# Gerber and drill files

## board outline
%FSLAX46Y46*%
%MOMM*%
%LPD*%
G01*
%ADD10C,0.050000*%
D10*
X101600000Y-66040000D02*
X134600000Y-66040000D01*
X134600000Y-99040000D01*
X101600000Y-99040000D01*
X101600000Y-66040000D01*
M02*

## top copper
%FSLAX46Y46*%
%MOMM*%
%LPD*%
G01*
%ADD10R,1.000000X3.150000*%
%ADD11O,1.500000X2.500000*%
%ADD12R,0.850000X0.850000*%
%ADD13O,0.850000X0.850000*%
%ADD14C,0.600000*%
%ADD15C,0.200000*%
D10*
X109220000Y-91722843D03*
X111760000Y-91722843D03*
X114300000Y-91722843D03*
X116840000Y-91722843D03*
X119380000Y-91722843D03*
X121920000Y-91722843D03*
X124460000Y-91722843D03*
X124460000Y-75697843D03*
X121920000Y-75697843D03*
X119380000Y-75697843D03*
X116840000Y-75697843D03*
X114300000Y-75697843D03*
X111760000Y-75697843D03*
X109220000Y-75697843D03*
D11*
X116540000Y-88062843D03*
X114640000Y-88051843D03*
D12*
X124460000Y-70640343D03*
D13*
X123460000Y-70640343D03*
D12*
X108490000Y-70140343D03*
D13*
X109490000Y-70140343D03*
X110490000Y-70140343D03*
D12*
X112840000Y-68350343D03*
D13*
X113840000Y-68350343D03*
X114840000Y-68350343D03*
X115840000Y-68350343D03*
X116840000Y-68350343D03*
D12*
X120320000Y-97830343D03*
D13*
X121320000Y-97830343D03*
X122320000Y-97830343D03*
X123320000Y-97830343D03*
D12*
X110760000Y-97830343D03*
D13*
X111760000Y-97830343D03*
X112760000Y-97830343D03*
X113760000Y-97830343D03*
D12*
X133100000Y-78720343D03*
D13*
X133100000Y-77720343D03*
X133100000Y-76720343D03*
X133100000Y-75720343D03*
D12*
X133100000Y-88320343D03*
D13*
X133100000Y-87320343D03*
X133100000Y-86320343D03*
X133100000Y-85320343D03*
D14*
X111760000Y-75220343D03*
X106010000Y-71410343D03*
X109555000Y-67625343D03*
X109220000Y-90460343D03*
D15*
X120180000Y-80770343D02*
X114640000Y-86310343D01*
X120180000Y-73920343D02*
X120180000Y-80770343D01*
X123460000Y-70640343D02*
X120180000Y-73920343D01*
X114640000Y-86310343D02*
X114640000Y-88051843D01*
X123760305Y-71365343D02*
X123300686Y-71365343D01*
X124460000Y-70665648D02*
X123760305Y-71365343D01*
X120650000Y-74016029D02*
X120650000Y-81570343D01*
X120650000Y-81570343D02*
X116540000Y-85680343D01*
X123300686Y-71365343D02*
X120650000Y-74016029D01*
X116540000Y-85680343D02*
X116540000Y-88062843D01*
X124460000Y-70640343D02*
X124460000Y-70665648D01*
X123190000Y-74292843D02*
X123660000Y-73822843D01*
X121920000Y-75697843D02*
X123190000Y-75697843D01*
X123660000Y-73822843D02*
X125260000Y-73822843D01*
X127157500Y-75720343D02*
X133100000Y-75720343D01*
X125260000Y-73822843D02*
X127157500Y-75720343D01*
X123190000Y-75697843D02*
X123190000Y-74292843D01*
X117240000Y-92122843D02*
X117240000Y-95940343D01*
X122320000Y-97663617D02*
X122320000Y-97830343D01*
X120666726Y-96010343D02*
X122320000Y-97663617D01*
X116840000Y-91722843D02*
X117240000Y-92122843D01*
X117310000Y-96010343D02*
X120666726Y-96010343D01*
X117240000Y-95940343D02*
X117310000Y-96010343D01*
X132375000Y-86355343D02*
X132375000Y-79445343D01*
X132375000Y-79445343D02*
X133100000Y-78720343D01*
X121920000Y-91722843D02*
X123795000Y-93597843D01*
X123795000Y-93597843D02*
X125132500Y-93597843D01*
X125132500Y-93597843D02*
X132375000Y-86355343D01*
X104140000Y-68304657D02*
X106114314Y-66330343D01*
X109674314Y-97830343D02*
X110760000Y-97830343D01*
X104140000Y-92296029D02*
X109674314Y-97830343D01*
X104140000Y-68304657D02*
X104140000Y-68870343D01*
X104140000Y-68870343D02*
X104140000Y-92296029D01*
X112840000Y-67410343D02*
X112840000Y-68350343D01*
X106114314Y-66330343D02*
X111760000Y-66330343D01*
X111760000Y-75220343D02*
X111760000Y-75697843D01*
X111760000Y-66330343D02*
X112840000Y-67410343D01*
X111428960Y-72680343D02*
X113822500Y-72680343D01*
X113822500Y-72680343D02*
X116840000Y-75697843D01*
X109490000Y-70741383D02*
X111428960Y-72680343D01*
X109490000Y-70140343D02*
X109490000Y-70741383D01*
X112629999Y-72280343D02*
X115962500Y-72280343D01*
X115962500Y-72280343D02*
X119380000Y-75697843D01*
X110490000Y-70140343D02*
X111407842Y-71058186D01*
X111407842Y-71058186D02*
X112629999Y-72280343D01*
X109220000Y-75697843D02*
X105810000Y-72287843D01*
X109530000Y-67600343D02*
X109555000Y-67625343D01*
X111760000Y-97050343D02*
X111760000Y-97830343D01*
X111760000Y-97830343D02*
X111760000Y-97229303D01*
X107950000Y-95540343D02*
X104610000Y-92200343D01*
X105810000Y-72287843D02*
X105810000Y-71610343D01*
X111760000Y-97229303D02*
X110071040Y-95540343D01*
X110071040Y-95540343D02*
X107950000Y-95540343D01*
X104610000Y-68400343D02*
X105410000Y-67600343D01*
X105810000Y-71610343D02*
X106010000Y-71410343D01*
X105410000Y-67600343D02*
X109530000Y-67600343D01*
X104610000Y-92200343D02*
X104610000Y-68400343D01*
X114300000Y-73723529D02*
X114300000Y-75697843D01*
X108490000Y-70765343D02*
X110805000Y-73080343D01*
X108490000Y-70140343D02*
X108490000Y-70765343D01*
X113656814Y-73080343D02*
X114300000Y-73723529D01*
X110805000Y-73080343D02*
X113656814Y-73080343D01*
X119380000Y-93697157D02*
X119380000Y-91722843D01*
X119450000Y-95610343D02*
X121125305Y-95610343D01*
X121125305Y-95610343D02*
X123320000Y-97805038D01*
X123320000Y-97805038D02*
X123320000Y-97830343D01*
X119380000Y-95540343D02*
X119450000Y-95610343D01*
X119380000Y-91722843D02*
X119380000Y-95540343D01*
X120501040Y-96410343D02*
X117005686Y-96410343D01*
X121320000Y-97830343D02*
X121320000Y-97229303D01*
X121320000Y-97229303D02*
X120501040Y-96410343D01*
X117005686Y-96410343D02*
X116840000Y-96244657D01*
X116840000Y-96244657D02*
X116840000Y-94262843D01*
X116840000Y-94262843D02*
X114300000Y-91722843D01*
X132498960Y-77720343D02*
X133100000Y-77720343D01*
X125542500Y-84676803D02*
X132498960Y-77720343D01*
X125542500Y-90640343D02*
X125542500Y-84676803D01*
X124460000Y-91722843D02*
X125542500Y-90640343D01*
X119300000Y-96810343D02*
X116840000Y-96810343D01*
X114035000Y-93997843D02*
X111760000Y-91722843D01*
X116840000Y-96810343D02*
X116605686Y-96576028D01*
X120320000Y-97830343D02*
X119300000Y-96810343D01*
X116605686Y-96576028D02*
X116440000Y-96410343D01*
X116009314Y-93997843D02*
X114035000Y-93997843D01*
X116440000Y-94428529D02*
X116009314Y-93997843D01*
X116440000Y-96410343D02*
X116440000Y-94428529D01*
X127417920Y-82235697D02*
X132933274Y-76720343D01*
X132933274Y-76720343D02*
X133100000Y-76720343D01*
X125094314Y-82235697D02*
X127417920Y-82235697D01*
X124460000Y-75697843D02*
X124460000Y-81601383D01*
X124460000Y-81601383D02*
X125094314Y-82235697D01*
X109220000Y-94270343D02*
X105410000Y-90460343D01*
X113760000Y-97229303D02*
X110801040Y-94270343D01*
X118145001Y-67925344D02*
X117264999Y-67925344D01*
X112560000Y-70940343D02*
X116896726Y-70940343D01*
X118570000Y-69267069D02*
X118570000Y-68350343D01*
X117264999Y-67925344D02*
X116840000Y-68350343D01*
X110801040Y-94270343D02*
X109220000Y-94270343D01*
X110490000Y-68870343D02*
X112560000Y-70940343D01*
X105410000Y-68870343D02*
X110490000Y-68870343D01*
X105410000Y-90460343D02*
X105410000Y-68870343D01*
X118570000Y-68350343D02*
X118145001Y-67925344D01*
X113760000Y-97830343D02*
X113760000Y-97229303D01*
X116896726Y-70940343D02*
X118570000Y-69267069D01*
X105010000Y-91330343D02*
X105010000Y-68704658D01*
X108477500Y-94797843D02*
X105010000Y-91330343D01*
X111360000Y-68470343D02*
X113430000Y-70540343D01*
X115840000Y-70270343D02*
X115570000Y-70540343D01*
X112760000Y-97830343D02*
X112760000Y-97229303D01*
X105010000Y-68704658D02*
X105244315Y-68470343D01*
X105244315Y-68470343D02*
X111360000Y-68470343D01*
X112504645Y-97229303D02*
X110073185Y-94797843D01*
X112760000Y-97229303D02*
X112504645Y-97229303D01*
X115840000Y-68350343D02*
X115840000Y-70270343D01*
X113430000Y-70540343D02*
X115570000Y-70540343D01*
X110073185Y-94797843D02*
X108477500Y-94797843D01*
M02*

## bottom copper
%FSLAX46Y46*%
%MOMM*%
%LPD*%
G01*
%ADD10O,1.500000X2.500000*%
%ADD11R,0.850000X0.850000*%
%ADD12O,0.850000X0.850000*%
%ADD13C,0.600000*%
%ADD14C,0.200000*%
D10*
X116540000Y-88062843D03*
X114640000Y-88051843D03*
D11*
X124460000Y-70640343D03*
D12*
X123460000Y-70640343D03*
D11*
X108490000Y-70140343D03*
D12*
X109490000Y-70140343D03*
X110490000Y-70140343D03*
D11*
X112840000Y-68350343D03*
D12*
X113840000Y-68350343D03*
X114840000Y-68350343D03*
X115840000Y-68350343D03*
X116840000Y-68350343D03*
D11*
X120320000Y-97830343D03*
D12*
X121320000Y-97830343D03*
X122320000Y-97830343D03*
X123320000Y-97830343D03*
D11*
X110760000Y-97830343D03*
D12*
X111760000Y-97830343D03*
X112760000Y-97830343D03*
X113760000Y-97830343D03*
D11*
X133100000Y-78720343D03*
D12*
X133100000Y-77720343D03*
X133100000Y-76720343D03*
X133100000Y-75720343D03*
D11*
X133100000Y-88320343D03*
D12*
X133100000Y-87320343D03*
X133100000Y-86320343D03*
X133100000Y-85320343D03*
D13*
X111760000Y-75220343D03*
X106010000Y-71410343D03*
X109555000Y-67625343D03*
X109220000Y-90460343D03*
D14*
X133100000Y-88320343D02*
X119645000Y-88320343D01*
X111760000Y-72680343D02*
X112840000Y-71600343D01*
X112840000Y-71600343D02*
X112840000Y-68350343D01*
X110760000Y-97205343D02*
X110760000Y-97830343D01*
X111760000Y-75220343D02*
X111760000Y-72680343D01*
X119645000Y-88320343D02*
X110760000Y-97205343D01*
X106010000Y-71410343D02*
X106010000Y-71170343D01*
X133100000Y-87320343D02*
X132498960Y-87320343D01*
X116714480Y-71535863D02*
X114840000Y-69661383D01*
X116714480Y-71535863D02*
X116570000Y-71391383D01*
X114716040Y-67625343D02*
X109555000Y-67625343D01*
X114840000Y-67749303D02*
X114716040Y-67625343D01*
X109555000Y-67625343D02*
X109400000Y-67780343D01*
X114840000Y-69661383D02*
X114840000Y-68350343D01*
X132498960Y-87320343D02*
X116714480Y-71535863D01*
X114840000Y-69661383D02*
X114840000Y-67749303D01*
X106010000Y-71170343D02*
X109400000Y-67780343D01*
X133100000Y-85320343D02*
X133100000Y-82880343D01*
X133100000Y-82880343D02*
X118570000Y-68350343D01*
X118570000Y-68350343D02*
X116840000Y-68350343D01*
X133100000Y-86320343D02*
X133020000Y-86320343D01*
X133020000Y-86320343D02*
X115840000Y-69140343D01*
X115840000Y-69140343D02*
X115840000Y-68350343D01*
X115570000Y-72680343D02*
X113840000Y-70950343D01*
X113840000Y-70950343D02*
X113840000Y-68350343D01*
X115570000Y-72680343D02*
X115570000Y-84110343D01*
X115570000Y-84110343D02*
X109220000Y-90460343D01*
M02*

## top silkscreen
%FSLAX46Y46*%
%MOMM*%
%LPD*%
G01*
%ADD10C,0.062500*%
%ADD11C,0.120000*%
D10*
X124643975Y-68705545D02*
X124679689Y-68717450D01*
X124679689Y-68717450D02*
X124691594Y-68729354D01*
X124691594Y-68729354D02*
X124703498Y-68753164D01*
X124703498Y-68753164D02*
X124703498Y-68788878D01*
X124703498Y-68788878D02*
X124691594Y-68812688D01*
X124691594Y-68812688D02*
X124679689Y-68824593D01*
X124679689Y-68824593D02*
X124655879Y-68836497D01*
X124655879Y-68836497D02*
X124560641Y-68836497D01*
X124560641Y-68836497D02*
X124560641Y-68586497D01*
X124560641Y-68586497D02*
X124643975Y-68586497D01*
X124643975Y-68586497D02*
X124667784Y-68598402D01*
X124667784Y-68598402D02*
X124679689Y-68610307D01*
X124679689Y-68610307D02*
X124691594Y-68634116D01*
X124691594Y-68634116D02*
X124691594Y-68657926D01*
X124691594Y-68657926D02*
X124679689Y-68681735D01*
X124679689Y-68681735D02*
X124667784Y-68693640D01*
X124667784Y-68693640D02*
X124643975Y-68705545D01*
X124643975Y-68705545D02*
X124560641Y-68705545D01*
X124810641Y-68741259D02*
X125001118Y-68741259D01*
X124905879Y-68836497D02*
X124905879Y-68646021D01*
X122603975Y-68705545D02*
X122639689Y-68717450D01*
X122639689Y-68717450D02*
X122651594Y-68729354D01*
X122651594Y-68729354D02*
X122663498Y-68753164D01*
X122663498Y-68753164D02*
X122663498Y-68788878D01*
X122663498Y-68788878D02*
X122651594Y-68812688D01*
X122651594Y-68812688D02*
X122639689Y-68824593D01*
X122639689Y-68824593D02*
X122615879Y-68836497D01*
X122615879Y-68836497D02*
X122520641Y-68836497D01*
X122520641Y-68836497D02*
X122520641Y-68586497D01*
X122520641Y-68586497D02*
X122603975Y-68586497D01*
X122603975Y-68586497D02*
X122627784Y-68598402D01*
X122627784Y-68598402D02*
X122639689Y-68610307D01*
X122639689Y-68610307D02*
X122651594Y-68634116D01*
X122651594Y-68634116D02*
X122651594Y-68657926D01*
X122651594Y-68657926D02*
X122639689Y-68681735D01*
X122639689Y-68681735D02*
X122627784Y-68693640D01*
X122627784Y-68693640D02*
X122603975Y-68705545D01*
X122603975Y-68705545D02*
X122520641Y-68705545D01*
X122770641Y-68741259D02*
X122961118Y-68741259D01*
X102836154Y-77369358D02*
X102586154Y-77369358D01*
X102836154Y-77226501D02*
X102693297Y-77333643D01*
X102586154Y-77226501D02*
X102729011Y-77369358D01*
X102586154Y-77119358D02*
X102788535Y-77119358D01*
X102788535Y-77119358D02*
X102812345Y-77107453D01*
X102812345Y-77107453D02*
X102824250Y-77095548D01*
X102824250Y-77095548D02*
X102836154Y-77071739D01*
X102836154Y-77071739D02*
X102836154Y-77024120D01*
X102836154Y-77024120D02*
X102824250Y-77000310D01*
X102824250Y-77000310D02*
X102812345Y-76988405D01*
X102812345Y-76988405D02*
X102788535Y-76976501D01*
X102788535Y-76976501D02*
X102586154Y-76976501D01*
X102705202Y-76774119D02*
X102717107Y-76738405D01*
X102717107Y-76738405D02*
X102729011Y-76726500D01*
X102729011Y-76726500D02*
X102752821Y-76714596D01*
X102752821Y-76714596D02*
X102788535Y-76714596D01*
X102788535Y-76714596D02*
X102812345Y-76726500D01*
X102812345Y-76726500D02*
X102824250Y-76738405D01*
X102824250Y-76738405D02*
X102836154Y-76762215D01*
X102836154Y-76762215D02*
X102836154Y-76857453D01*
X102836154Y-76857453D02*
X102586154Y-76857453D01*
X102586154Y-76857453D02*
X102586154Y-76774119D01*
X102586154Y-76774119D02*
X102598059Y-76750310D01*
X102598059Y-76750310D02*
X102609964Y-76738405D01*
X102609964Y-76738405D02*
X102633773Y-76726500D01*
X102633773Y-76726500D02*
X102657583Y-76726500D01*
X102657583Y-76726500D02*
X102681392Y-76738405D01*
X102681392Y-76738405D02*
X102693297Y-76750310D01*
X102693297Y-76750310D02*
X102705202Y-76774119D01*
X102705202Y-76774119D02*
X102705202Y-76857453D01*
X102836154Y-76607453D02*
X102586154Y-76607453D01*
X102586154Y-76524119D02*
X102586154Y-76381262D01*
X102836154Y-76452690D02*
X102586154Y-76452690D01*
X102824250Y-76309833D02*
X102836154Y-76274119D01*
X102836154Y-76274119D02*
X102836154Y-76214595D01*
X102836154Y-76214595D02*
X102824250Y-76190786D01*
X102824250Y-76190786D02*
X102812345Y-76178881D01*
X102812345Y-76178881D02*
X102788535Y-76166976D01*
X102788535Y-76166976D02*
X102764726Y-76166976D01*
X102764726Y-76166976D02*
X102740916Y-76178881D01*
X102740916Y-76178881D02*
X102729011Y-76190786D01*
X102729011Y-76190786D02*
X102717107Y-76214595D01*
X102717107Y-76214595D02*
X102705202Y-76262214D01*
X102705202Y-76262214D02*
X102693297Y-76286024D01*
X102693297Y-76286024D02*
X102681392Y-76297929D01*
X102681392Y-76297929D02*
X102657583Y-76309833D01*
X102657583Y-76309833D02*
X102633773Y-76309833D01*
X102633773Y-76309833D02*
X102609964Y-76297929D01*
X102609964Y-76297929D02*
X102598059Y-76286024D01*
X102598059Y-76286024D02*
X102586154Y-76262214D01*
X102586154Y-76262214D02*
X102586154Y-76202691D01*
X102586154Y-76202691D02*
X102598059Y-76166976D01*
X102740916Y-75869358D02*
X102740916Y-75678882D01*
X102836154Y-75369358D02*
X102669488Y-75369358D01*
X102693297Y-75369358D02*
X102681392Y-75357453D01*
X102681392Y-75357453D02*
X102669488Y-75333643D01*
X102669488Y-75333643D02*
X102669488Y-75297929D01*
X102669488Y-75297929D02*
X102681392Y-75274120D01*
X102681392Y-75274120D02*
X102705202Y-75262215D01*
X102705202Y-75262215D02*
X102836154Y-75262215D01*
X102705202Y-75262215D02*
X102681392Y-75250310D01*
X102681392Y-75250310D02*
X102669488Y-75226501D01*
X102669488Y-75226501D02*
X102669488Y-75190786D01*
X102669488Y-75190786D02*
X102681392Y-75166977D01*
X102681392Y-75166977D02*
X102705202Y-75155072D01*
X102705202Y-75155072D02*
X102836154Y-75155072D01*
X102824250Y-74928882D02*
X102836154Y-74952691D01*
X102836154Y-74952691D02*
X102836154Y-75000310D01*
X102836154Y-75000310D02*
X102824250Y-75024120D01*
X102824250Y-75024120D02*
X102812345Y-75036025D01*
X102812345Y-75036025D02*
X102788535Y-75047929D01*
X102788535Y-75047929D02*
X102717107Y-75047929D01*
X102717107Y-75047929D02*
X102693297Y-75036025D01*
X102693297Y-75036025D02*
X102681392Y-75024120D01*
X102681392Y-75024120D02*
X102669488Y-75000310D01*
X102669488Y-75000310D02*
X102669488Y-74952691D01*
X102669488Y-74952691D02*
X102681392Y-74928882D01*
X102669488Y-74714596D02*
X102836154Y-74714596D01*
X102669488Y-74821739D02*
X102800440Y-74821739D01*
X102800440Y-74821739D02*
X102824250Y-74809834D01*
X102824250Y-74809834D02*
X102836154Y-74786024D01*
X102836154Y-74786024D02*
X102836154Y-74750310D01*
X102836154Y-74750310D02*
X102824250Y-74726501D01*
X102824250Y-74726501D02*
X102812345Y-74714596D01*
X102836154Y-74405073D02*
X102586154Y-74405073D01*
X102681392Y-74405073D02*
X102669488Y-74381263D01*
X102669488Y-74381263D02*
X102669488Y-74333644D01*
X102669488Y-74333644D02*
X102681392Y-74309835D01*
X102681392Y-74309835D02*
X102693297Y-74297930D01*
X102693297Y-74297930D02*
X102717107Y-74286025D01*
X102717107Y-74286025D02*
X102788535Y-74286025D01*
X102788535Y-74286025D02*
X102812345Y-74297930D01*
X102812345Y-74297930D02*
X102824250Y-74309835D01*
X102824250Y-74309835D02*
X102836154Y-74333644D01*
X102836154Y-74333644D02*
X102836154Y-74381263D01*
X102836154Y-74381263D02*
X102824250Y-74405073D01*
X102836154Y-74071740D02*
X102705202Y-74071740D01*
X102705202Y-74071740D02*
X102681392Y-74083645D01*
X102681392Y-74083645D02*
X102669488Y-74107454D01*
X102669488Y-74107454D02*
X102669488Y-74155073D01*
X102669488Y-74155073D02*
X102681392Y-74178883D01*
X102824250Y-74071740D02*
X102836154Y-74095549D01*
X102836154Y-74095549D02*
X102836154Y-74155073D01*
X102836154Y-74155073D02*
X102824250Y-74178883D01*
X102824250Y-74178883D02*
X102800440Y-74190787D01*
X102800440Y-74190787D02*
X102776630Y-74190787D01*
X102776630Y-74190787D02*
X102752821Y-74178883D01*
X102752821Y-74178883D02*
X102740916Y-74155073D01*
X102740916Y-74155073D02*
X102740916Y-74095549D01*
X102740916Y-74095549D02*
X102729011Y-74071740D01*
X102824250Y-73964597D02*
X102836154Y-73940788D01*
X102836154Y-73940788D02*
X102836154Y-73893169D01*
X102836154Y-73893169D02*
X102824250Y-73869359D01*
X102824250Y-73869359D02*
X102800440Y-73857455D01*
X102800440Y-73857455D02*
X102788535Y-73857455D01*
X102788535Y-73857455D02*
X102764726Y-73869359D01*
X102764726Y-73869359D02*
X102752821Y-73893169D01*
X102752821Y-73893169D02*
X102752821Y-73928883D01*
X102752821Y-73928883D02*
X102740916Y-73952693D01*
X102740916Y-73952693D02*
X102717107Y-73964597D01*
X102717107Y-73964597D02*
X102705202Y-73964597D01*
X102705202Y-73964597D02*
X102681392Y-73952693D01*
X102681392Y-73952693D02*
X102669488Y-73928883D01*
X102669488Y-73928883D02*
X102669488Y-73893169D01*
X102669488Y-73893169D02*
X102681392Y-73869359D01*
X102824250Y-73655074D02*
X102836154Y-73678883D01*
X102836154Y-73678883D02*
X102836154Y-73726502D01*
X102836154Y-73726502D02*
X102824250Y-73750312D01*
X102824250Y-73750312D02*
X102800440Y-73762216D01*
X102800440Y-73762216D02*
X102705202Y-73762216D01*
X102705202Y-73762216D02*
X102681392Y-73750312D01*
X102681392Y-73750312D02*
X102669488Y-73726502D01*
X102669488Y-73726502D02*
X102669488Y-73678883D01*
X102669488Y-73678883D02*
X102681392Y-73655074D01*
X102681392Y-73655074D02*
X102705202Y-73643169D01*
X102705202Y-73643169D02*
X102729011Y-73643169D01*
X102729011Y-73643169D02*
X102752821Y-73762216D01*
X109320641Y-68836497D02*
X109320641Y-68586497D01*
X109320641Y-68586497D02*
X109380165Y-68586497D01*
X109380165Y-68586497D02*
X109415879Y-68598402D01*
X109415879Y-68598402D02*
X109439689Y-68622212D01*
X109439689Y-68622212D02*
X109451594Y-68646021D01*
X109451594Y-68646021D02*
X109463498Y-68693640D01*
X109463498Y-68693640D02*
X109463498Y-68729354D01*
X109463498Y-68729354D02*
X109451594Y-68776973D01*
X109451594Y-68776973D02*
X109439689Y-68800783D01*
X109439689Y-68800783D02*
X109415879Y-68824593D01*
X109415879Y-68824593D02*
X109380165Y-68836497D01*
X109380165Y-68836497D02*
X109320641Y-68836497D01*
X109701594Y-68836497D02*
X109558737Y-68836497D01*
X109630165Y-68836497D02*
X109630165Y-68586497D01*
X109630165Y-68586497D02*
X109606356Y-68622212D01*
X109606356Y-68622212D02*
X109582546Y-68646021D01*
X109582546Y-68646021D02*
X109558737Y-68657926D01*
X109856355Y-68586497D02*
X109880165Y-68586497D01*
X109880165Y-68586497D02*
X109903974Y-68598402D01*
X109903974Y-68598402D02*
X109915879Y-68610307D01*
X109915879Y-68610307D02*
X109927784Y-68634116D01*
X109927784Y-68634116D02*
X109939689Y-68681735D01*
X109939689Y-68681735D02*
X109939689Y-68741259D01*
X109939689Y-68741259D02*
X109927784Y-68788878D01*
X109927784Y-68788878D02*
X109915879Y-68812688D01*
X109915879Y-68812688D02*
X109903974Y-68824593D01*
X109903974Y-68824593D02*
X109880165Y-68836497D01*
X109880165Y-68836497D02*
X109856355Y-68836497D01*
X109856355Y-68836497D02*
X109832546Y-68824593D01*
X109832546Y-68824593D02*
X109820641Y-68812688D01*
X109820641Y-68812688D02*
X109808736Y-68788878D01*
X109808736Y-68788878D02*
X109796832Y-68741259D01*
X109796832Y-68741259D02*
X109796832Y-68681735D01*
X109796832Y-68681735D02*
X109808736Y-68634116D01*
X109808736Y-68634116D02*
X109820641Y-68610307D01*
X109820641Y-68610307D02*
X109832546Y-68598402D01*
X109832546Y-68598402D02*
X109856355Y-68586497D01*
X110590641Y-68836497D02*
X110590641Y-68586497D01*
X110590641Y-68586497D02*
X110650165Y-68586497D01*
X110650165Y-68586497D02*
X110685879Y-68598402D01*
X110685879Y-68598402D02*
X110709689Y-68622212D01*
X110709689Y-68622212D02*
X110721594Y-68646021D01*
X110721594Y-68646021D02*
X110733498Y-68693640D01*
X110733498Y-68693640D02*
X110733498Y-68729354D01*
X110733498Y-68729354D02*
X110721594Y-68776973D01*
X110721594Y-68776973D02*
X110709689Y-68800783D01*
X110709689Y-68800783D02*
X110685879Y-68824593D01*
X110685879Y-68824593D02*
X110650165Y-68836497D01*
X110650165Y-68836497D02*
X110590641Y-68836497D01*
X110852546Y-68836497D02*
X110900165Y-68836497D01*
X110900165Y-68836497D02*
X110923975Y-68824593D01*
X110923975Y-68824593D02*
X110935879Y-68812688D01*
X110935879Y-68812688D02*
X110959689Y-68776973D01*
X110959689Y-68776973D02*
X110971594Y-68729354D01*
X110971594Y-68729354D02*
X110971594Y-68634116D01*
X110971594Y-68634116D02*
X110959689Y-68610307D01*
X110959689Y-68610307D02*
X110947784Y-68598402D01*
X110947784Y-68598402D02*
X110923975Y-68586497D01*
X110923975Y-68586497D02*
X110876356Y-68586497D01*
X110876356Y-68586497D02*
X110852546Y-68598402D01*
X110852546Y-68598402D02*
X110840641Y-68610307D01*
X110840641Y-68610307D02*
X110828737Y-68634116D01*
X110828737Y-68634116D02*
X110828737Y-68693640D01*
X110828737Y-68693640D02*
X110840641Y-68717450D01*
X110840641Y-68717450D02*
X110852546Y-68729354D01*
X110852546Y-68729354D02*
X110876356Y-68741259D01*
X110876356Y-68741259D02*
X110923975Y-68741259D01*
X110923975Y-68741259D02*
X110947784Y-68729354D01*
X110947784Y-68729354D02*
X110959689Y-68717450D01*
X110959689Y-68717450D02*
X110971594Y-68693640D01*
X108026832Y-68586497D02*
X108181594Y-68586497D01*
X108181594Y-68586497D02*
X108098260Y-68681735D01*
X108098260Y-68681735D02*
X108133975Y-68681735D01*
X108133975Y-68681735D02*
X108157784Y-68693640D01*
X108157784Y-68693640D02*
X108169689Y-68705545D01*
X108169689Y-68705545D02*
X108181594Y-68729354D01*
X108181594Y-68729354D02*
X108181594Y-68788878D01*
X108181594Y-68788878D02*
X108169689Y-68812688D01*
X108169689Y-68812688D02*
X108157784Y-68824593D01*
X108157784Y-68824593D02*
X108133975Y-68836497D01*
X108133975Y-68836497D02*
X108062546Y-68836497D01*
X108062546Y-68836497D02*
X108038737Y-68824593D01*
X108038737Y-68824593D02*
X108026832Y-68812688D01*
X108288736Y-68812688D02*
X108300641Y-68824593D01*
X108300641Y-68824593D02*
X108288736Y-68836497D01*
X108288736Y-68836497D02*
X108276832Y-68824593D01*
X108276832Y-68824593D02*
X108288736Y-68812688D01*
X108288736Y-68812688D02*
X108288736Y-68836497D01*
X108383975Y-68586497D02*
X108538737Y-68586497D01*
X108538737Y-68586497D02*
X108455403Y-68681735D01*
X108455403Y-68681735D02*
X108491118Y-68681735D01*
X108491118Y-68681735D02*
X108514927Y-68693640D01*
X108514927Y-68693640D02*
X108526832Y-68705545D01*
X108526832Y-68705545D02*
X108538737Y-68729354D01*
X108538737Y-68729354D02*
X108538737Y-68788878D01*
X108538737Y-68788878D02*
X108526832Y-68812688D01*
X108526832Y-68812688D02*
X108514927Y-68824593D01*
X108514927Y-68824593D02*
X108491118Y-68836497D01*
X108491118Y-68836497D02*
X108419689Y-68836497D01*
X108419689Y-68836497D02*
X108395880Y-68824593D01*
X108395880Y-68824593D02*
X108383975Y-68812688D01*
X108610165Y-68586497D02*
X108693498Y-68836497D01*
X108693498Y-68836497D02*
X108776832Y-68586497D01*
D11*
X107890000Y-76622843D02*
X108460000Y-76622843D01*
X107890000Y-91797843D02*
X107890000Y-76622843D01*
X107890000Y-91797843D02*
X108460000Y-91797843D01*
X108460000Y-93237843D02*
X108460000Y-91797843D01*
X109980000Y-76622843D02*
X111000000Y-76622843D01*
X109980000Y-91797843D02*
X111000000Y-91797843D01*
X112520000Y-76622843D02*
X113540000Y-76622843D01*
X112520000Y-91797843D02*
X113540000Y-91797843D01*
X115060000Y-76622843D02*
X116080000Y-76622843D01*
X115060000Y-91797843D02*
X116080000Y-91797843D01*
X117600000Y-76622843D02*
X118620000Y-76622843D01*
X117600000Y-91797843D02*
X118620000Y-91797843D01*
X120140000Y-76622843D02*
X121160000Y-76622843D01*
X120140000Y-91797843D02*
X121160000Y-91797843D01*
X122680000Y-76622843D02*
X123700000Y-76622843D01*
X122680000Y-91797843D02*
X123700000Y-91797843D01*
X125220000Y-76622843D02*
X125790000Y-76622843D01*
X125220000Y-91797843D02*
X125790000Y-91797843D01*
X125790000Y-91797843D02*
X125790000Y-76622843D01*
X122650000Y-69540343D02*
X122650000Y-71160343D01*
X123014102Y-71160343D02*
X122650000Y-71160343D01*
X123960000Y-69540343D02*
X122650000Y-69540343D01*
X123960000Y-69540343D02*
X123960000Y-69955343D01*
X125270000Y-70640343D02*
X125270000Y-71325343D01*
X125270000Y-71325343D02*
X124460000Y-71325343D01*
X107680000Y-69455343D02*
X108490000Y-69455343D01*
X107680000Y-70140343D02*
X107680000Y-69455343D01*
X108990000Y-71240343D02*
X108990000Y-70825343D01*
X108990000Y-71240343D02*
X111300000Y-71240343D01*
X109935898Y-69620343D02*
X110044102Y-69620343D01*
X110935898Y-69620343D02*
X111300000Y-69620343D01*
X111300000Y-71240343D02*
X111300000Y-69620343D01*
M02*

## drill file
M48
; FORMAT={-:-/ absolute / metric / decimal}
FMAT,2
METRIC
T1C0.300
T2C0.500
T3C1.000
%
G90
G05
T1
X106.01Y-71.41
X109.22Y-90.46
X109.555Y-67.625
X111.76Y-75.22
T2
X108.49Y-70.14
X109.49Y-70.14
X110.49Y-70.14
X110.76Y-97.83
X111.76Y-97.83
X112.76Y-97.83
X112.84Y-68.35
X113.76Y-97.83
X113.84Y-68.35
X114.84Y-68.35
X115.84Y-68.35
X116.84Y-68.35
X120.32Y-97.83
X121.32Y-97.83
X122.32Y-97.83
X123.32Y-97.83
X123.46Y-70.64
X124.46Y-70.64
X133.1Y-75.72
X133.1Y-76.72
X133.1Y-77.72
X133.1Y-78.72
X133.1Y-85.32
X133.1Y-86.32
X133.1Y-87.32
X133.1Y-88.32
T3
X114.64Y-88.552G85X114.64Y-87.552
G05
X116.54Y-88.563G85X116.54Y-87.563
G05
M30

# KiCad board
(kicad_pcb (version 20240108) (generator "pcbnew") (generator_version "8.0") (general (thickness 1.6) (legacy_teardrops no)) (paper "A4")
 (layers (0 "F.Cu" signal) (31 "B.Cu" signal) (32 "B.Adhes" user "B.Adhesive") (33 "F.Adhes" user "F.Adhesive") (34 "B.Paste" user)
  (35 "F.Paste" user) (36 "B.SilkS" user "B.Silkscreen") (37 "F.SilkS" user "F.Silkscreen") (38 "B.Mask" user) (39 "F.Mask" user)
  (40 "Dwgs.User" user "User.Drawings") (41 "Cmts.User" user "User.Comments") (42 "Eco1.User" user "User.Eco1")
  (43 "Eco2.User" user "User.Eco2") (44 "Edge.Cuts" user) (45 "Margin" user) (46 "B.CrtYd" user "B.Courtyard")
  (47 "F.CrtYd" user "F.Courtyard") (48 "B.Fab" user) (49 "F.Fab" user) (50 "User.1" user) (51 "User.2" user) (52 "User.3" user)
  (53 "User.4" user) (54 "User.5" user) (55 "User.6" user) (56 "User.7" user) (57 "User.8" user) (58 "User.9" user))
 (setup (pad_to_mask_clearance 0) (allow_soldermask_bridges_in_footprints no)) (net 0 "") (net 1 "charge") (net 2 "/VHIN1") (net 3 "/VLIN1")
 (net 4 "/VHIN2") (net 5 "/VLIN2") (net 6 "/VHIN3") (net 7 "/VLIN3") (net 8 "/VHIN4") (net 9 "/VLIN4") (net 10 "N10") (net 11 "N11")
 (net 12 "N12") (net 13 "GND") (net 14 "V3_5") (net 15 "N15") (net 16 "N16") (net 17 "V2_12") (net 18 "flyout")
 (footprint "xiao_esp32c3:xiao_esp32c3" (layer "F.Cu") (at 118.64 83.122843 90)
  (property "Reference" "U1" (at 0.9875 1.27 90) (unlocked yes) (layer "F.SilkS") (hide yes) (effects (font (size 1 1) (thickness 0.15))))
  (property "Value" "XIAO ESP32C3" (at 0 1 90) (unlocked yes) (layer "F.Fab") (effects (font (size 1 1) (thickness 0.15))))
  (fp_line (start 6.5 -10.75) (end 6.5 -10.18) (stroke (width 0.12) (type solid)) (layer "F.SilkS"))
  (fp_line (start -8.675 -10.75) (end 6.5 -10.75) (stroke (width 0.12) (type solid)) (layer "F.SilkS"))
  (fp_line (start -8.675 -10.75) (end -8.675 -10.18) (stroke (width 0.12) (type solid)) (layer "F.SilkS"))
  (fp_line (start -10.115 -10.18) (end -8.675 -10.18) (stroke (width 0.12) (type solid)) (layer "F.SilkS"))
  (fp_line (start 6.5 -8.66) (end 6.5 -7.64) (stroke (width 0.12) (type solid)) (layer "F.SilkS"))
  (fp_line (start -8.675 -8.66) (end -8.675 -7.64) (stroke (width 0.12) (type solid)) (layer "F.SilkS"))
  (fp_line (start 6.5 -6.12) (end 6.5 -5.1) (stroke (width 0.12) (type solid)) (layer "F.SilkS"))
  (fp_line (start -8.675 -6.12) (end -8.675 -5.1) (stroke (width 0.12) (type solid)) (layer "F.SilkS"))
  (fp_line (start 6.5 -3.58) (end 6.5 -2.56) (stroke (width 0.12) (type solid)) (layer "F.SilkS"))
  (fp_line (start -8.675 -3.58) (end -8.675 -2.56) (stroke (width 0.12) (type solid)) (layer "F.SilkS"))
  (fp_line (start 6.5 -1.04) (end 6.5 -0.02) (stroke (width 0.12) (type solid)) (layer "F.SilkS"))
  (fp_line (start -8.675 -1.04) (end -8.675 -0.02) (stroke (width 0.12) (type solid)) (layer "F.SilkS"))
  (fp_line (start 6.5 1.5) (end 6.5 2.52) (stroke (width 0.12) (type solid)) (layer "F.SilkS"))
  (fp_line (start -8.675 1.5) (end -8.675 2.52) (stroke (width 0.12) (type solid)) (layer "F.SilkS"))
  (fp_line (start 6.5 4.04) (end 6.5 5.06) (stroke (width 0.12) (type solid)) (layer "F.SilkS"))
  (fp_line (start -8.675 4.04) (end -8.675 5.06) (stroke (width 0.12) (type solid)) (layer "F.SilkS"))
  (fp_line (start 6.5 6.58) (end 6.5 7.15) (stroke (width 0.12) (type solid)) (layer "F.SilkS"))
  (fp_line (start -8.675 6.58) (end -8.675 7.15) (stroke (width 0.12) (type solid)) (layer "F.SilkS"))
  (fp_line (start -8.675 7.15) (end 6.5 7.15) (stroke (width 0.12) (type solid)) (layer "F.SilkS"))
  (pad "1" smd rect (at -8.6 -9.42 90) (size 3.15 1) (layers "F.Cu" "F.Paste" "F.Mask") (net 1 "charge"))
  (pad "2" smd rect (at -8.6 -6.88 90) (size 3.15 1) (layers "F.Cu" "F.Paste" "F.Mask") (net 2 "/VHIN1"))
  (pad "3" smd rect (at -8.6 -4.34 90) (size 3.15 1) (layers "F.Cu" "F.Paste" "F.Mask") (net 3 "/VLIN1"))
  (pad "4" smd rect (at -8.6 -1.8 90) (size 3.15 1) (layers "F.Cu" "F.Paste" "F.Mask") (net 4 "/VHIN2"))
  (pad "5" smd rect (at -8.6 0.74 90) (size 3.15 1) (layers "F.Cu" "F.Paste" "F.Mask") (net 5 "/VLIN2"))
  (pad "6" smd rect (at -8.6 3.28 90) (size 3.15 1) (layers "F.Cu" "F.Paste" "F.Mask") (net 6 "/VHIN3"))
  (pad "7" smd rect (at -8.6 5.82 90) (size 3.15 1) (layers "F.Cu" "F.Paste" "F.Mask") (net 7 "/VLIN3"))
  (pad "8" smd rect (at 7.425 5.82 90) (size 3.15 1) (layers "F.Cu" "F.Paste" "F.Mask") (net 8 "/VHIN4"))
  (pad "9" smd rect (at 7.425 3.28 90) (size 3.15 1) (layers "F.Cu" "F.Paste" "F.Mask") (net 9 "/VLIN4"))
  (pad "10" smd rect (at 7.425 0.74 90) (size 3.15 1) (layers "F.Cu" "F.Paste" "F.Mask") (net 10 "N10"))
  (pad "11" smd rect (at 7.425 -1.8 90) (size 3.15 1) (layers "F.Cu" "F.Paste" "F.Mask") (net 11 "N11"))
  (pad "12" smd rect (at 7.425 -4.34 90) (size 3.15 1) (layers "F.Cu" "F.Paste" "F.Mask") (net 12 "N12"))
  (pad "13" smd rect (at 7.425 -6.88 90) (size 3.15 1) (layers "F.Cu" "F.Paste" "F.Mask") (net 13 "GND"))
  (pad "14" smd rect (at 7.425 -9.42 90) (size 3.15 1) (layers "F.Cu" "F.Paste" "F.Mask") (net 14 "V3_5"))
  (pad "B+" thru_hole oval (at -4.94 -2.1 90) (size 2.5 1.5) (drill oval 2 1) (layers "*.Cu" "*.Mask") (remove_unused_layers no)
   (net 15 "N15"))
  (pad "B-" thru_hole oval (at -4.929 -4 90) (size 2.5 1.5) (drill oval 2 1) (layers "*.Cu" "*.Mask") (remove_unused_layers no)
   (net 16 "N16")))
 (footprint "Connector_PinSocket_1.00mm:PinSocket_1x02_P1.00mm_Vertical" (layer "F.Cu") (at 124.46 70.640343 -90)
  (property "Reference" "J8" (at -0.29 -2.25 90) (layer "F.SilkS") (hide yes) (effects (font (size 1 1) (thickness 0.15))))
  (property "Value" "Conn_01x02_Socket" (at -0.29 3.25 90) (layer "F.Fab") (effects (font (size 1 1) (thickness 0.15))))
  (fp_line (start -1.1 1.81) (end 0.52 1.81) (stroke (width 0.12) (type solid)) (layer "F.SilkS"))
  (fp_line (start 0.52 1.445898) (end 0.52 1.81) (stroke (width 0.12) (type solid)) (layer "F.SilkS"))
  (fp_line (start -1.1 0.5) (end -1.1 1.81) (stroke (width 0.12) (type solid)) (layer "F.SilkS"))
  (fp_line (start -1.1 0.5) (end -0.685 0.5) (stroke (width 0.12) (type solid)) (layer "F.SilkS"))
  (fp_line (start 0 -0.81) (end 0.685 -0.81) (stroke (width 0.12) (type solid)) (layer "F.SilkS"))
  (fp_line (start 0.685 -0.81) (end 0.685 0) (stroke (width 0.12) (type solid)) (layer "F.SilkS"))
  (pad "1" thru_hole rect (at 0 0 270) (size 0.85 0.85) (drill 0.5) (layers "*.Cu" "*.Mask") (remove_unused_layers no) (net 15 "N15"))
  (pad "2" thru_hole oval (at 0 1 270) (size 0.85 0.85) (drill 0.5) (layers "*.Cu" "*.Mask") (remove_unused_layers no) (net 16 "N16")))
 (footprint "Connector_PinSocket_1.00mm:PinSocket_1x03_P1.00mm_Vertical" (layer "F.Cu") (at 108.49 70.140343 90)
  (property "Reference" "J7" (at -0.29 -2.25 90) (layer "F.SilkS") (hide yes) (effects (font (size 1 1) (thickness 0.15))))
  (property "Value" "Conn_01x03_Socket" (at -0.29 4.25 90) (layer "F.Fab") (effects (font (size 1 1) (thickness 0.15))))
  (fp_line (start 0.685 -0.81) (end 0.685 0) (stroke (width 0.12) (type solid)) (layer "F.SilkS"))
  (fp_line (start 0 -0.81) (end 0.685 -0.81) (stroke (width 0.12) (type solid)) (layer "F.SilkS"))
  (fp_line (start -1.1 0.5) (end -0.685 0.5) (stroke (width 0.12) (type solid)) (layer "F.SilkS"))
  (fp_line (start -1.1 0.5) (end -1.1 2.81) (stroke (width 0.12) (type solid)) (layer "F.SilkS"))
  (fp_line (start 0.52 1.445898) (end 0.52 1.554102) (stroke (width 0.12) (type solid)) (layer "F.SilkS"))
  (fp_line (start 0.52 2.445898) (end 0.52 2.81) (stroke (width 0.12) (type solid)) (layer "F.SilkS"))
  (fp_line (start -1.1 2.81) (end 0.52 2.81) (stroke (width 0.12) (type solid)) (layer "F.SilkS"))
  (pad "1" thru_hole rect (at 0 0 90) (size 0.85 0.85) (drill 0.5) (layers "*.Cu" "*.Mask") (remove_unused_layers no) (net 12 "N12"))
  (pad "2" thru_hole oval (at 0 1 90) (size 0.85 0.85) (drill 0.5) (layers "*.Cu" "*.Mask") (remove_unused_layers no) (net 11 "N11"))
  (pad "3" thru_hole oval (at 0 2 90) (size 0.85 0.85) (drill 0.5) (layers "*.Cu" "*.Mask") (remove_unused_layers no) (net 10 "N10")))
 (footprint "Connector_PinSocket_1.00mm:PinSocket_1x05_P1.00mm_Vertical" (layer "B.Cu") (at 112.84 68.350343 -90)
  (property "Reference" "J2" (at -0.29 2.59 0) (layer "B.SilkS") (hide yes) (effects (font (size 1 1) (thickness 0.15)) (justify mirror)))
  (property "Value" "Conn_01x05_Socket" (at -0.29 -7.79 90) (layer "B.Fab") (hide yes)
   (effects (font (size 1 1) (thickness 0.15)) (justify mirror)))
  (pad "1" thru_hole rect (at 0 0 270) (size 0.85 0.85) (drill 0.5) (layers "*.Cu" "*.Mask") (remove_unused_layers no) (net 13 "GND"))
  (pad "2" thru_hole oval (at 0 -1 270) (size 0.85 0.85) (drill 0.5) (layers "*.Cu" "*.Mask") (remove_unused_layers no) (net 1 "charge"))
  (pad "3" thru_hole oval (at 0 -2 270) (size 0.85 0.85) (drill 0.5) (layers "*.Cu" "*.Mask") (remove_unused_layers no) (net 14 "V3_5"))
  (pad "4" thru_hole oval (at 0 -3 270) (size 0.85 0.85) (drill 0.5) (layers "*.Cu" "*.Mask") (remove_unused_layers no) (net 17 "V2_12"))
  (pad "5" thru_hole oval (at 0 -4 270) (size 0.85 0.85) (drill 0.5) (layers "*.Cu" "*.Mask") (remove_unused_layers no) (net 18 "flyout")))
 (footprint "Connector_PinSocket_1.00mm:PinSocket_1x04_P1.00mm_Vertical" (layer "B.Cu") (at 120.32 97.830343 -90)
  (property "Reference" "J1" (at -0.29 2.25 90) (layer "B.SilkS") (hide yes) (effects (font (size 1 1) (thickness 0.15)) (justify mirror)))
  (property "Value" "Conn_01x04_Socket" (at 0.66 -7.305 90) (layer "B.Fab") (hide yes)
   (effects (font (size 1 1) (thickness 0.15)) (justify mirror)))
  (pad "1" thru_hole rect (at 0 0 270) (size 0.85 0.85) (drill 0.5) (layers "*.Cu" "*.Mask") (remove_unused_layers no) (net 2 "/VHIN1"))
  (pad "2" thru_hole oval (at 0 -1 270) (size 0.85 0.85) (drill 0.5) (layers "*.Cu" "*.Mask") (remove_unused_layers no) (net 3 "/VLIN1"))
  (pad "3" thru_hole oval (at 0 -2 270) (size 0.85 0.85) (drill 0.5) (layers "*.Cu" "*.Mask") (remove_unused_layers no) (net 4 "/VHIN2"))
  (pad "4" thru_hole oval (at 0 -3 270) (size 0.85 0.85) (drill 0.5) (layers "*.Cu" "*.Mask") (remove_unused_layers no) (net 5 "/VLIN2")))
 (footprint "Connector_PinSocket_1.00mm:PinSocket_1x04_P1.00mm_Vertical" (layer "B.Cu") (at 110.76 97.830343 -90)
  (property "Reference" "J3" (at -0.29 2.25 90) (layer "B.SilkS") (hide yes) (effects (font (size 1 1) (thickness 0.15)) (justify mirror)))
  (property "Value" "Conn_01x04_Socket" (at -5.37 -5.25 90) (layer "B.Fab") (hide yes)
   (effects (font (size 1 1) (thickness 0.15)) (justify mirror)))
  (pad "1" thru_hole rect (at 0 0 270) (size 0.85 0.85) (drill 0.5) (layers "*.Cu" "*.Mask") (remove_unused_layers no) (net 13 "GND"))
  (pad "2" thru_hole oval (at 0 -1 270) (size 0.85 0.85) (drill 0.5) (layers "*.Cu" "*.Mask") (remove_unused_layers no) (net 14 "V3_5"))
  (pad "3" thru_hole oval (at 0 -2 270) (size 0.85 0.85) (drill 0.5) (layers "*.Cu" "*.Mask") (remove_unused_layers no) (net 17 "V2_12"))
  (pad "4" thru_hole oval (at 0 -3 270) (size 0.85 0.85) (drill 0.5) (layers "*.Cu" "*.Mask") (remove_unused_layers no) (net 18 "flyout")))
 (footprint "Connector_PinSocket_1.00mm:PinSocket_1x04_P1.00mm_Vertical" (layer "B.Cu") (at 133.1 78.720343)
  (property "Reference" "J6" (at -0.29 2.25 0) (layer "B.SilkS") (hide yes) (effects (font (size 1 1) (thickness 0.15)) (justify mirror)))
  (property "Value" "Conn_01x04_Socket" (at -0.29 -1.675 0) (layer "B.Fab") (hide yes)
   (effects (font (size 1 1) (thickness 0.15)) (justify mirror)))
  (pad "1" thru_hole rect (at 0 0) (size 0.85 0.85) (drill 0.5) (layers "*.Cu" "*.Mask") (remove_unused_layers no) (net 6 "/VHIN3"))
  (pad "2" thru_hole oval (at 0 -1) (size 0.85 0.85) (drill 0.5) (layers "*.Cu" "*.Mask") (remove_unused_layers no) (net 7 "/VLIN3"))
  (pad "3" thru_hole oval (at 0 -2) (size 0.85 0.85) (drill 0.5) (layers "*.Cu" "*.Mask") (remove_unused_layers no) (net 8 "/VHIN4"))
  (pad "4" thru_hole oval (at 0 -3) (size 0.85 0.85) (drill 0.5) (layers "*.Cu" "*.Mask") (remove_unused_layers no) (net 9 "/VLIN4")))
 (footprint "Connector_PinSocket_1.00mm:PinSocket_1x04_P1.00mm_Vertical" (layer "B.Cu") (at 133.1 88.320343)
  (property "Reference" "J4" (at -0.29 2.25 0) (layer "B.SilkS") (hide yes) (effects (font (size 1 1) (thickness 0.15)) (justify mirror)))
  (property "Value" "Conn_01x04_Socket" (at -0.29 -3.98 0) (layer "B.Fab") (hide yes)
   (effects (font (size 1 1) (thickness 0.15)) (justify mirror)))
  (pad "1" thru_hole rect (at 0 0) (size 0.85 0.85) (drill 0.5) (layers "*.Cu" "*.Mask") (remove_unused_layers no) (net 13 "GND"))
  (pad "2" thru_hole oval (at 0 -1) (size 0.85 0.85) (drill 0.5) (layers "*.Cu" "*.Mask") (remove_unused_layers no) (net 14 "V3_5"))
  (pad "3" thru_hole oval (at 0 -2) (size 0.85 0.85) (drill 0.5) (layers "*.Cu" "*.Mask") (remove_unused_layers no) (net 17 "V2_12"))
  (pad "4" thru_hole oval (at 0 -3) (size 0.85 0.85) (drill 0.5) (layers "*.Cu" "*.Mask") (remove_unused_layers no) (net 18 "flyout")))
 (gr_rect (start 101.6 66.04) (end 134.6 99.04) (stroke (width 0.05) (type default)) (fill none) (layer "Edge.Cuts"))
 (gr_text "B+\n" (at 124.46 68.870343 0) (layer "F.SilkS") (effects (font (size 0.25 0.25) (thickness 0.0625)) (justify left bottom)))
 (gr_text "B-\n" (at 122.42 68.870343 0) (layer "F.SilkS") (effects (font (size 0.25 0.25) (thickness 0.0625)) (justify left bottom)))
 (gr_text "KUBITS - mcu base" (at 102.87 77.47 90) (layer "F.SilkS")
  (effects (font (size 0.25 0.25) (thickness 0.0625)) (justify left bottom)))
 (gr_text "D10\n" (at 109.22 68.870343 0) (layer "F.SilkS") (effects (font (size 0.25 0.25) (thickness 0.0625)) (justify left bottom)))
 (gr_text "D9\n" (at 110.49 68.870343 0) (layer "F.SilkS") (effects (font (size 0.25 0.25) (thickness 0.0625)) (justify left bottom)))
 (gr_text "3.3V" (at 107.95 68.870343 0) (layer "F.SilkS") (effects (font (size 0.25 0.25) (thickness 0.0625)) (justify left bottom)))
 (segment (start 120.18 80.770343) (end 114.64 86.310343) (width 0.2) (layer "F.Cu") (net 16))
 (segment (start 120.18 73.920343) (end 120.18 80.770343) (width 0.2) (layer "F.Cu") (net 16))
 (segment (start 123.46 70.640343) (end 120.18 73.920343) (width 0.2) (layer "F.Cu") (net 16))
 (segment (start 114.64 86.310343) (end 114.64 88.051843) (width 0.2) (layer "F.Cu") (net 16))
 (segment (start 123.760305 71.365343) (end 123.300686 71.365343) (width 0.2) (layer "F.Cu") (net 15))
 (segment (start 124.46 70.665648) (end 123.760305 71.365343) (width 0.2) (layer "F.Cu") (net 15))
 (segment (start 120.65 74.016029) (end 120.65 81.570343) (width 0.2) (layer "F.Cu") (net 15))
 (segment (start 120.65 81.570343) (end 116.54 85.680343) (width 0.2) (layer "F.Cu") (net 15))
 (segment (start 123.300686 71.365343) (end 120.65 74.016029) (width 0.2) (layer "F.Cu") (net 15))
 (segment (start 116.54 85.680343) (end 116.54 88.062843) (width 0.2) (layer "F.Cu") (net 15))
 (segment (start 124.46 70.640343) (end 124.46 70.665648) (width 0.2) (layer "F.Cu") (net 15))
 (segment (start 123.19 74.292843) (end 123.66 73.822843) (width 0.2) (layer "F.Cu") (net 9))
 (segment (start 121.92 75.697843) (end 123.19 75.697843) (width 0.2) (layer "F.Cu") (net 9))
 (segment (start 123.66 73.822843) (end 125.26 73.822843) (width 0.2) (layer "F.Cu") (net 9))
 (segment (start 127.1575 75.720343) (end 133.1 75.720343) (width 0.2) (layer "F.Cu") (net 9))
 (segment (start 125.26 73.822843) (end 127.1575 75.720343) (width 0.2) (layer "F.Cu") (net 9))
 (segment (start 123.19 75.697843) (end 123.19 74.292843) (width 0.2) (layer "F.Cu") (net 9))
 (segment (start 117.24 92.122843) (end 117.24 95.940343) (width 0.2) (layer "F.Cu") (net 4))
 (segment (start 122.32 97.663617) (end 122.32 97.830343) (width 0.2) (layer "F.Cu") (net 4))
 (segment (start 120.666726 96.010343) (end 122.32 97.663617) (width 0.2) (layer "F.Cu") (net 4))
 (segment (start 116.84 91.722843) (end 117.24 92.122843) (width 0.2) (layer "F.Cu") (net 4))
 (segment (start 117.31 96.010343) (end 120.666726 96.010343) (width 0.2) (layer "F.Cu") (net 4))
 (segment (start 117.24 95.940343) (end 117.31 96.010343) (width 0.2) (layer "F.Cu") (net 4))
 (segment (start 132.375 86.355343) (end 132.375 79.445343) (width 0.2) (layer "F.Cu") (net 6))
 (segment (start 132.375 79.445343) (end 133.1 78.720343) (width 0.2) (layer "F.Cu") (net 6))
 (segment (start 121.92 91.722843) (end 123.795 93.597843) (width 0.2) (layer "F.Cu") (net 6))
 (segment (start 123.795 93.597843) (end 125.1325 93.597843) (width 0.2) (layer "F.Cu") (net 6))
 (segment (start 125.1325 93.597843) (end 132.375 86.355343) (width 0.2) (layer "F.Cu") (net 6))
 (segment (start 104.14 68.304657) (end 106.114314 66.330343) (width 0.2) (layer "F.Cu") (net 13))
 (segment (start 109.674314 97.830343) (end 110.76 97.830343) (width 0.2) (layer "F.Cu") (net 13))
 (segment (start 104.14 92.296029) (end 109.674314 97.830343) (width 0.2) (layer "F.Cu") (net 13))
 (segment (start 104.14 68.304657) (end 104.14 68.870343) (width 0.2) (layer "F.Cu") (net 13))
 (segment (start 104.14 68.870343) (end 104.14 92.296029) (width 0.2) (layer "F.Cu") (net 13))
 (segment (start 112.84 67.410343) (end 112.84 68.350343) (width 0.2) (layer "F.Cu") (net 13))
 (segment (start 106.114314 66.330343) (end 111.76 66.330343) (width 0.2) (layer "F.Cu") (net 13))
 (segment (start 111.76 75.220343) (end 111.76 75.697843) (width 0.2) (layer "F.Cu") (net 13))
 (segment (start 111.76 66.330343) (end 112.84 67.410343) (width 0.2) (layer "F.Cu") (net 13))
 (via (at 111.76 75.220343) (size 0.6) (drill 0.3) (layers "F.Cu" "B.Cu") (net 13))
 (segment (start 133.1 88.320343) (end 119.645 88.320343) (width 0.2) (layer "B.Cu") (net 13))
 (segment (start 111.76 72.680343) (end 112.84 71.600343) (width 0.2) (layer "B.Cu") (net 13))
 (segment (start 112.84 71.600343) (end 112.84 68.350343) (width 0.2) (layer "B.Cu") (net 13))
 (segment (start 110.76 97.205343) (end 110.76 97.830343) (width 0.2) (layer "B.Cu") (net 13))
 (segment (start 111.76 75.220343) (end 111.76 72.680343) (width 0.2) (layer "B.Cu") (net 13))
 (segment (start 119.645 88.320343) (end 110.76 97.205343) (width 0.2) (layer "B.Cu") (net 13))
 (segment (start 111.42896 72.680343) (end 113.8225 72.680343) (width 0.2) (layer "F.Cu") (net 11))
 (segment (start 113.8225 72.680343) (end 116.84 75.697843) (width 0.2) (layer "F.Cu") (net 11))
 (segment (start 109.49 70.741383) (end 111.42896 72.680343) (width 0.2) (layer "F.Cu") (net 11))
 (segment (start 109.49 70.140343) (end 109.49 70.741383) (width 0.2) (layer "F.Cu") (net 11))
 (segment (start 112.629999 72.280343) (end 115.9625 72.280343) (width 0.2) (layer "F.Cu") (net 10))
 (segment (start 115.9625 72.280343) (end 119.38 75.697843) (width 0.2) (layer "F.Cu") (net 10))
 (segment (start 110.49 70.140343) (end 111.407842 71.058186) (width 0.2) (layer "F.Cu") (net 10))
 (segment (start 111.407842 71.058186) (end 112.629999 72.280343) (width 0.2) (layer "F.Cu") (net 10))
 (segment (start 109.22 75.697843) (end 105.81 72.287843) (width 0.2) (layer "F.Cu") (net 14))
 (segment (start 109.53 67.600343) (end 109.555 67.625343) (width 0.2) (layer "F.Cu") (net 14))
 (segment (start 111.76 97.050343) (end 111.76 97.830343) (width 0.2) (layer "F.Cu") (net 14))
 (segment (start 111.76 97.830343) (end 111.76 97.229303) (width 0.2) (layer "F.Cu") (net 14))
 (segment (start 107.95 95.540343) (end 104.61 92.200343) (width 0.2) (layer "F.Cu") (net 14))
 (segment (start 105.81 72.287843) (end 105.81 71.610343) (width 0.2) (layer "F.Cu") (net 14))
 (segment (start 111.76 97.229303) (end 110.07104 95.540343) (width 0.2) (layer "F.Cu") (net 14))
 (segment (start 110.07104 95.540343) (end 107.95 95.540343) (width 0.2) (layer "F.Cu") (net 14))
 (segment (start 104.61 68.400343) (end 105.41 67.600343) (width 0.2) (layer "F.Cu") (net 14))
 (segment (start 105.81 71.610343) (end 106.01 71.410343) (width 0.2) (layer "F.Cu") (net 14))
 (segment (start 105.41 67.600343) (end 109.53 67.600343) (width 0.2) (layer "F.Cu") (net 14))
 (segment (start 104.61 92.200343) (end 104.61 68.400343) (width 0.2) (layer "F.Cu") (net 14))
 (via (at 106.01 71.410343) (size 0.6) (drill 0.3) (layers "F.Cu" "B.Cu") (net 14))
 (via (at 109.555 67.625343) (size 0.6) (drill 0.3) (layers "F.Cu" "B.Cu") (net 14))
 (segment (start 106.01 71.410343) (end 106.01 71.170343) (width 0.2) (layer "B.Cu") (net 14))
 (segment (start 133.1 87.320343) (end 132.49896 87.320343) (width 0.2) (layer "B.Cu") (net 14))
 (segment (start 116.71448 71.535863) (end 114.84 69.661383) (width 0.2) (layer "B.Cu") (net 14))
 (segment (start 116.71448 71.535863) (end 116.57 71.391383) (width 0.2) (layer "B.Cu") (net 14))
 (segment (start 114.71604 67.625343) (end 109.555 67.625343) (width 0.2) (layer "B.Cu") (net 14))
 (segment (start 114.84 67.749303) (end 114.71604 67.625343) (width 0.2) (layer "B.Cu") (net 14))
 (segment (start 109.555 67.625343) (end 109.4 67.780343) (width 0.2) (layer "B.Cu") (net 14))
 (segment (start 114.84 69.661383) (end 114.84 68.350343) (width 0.2) (layer "B.Cu") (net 14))
 (segment (start 132.49896 87.320343) (end 116.71448 71.535863) (width 0.2) (layer "B.Cu") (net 14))
 (segment (start 114.84 69.661383) (end 114.84 67.749303) (width 0.2) (layer "B.Cu") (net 14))
 (segment (start 106.01 71.170343) (end 109.4 67.780343) (width 0.2) (layer "B.Cu") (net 14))
 (segment (start 114.3 73.723529) (end 114.3 75.697843) (width 0.2) (layer "F.Cu") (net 12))
 (segment (start 108.49 70.765343) (end 110.805 73.080343) (width 0.2) (layer "F.Cu") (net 12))
 (segment (start 108.49 70.140343) (end 108.49 70.765343) (width 0.2) (layer "F.Cu") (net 12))
 (segment (start 113.656814 73.080343) (end 114.3 73.723529) (width 0.2) (layer "F.Cu") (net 12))
 (segment (start 110.805 73.080343) (end 113.656814 73.080343) (width 0.2) (layer "F.Cu") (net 12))
 (segment (start 119.38 93.697157) (end 119.38 91.722843) (width 0.2) (layer "F.Cu") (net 5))
 (segment (start 119.45 95.610343) (end 121.125305 95.610343) (width 0.2) (layer "F.Cu") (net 5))
 (segment (start 121.125305 95.610343) (end 123.32 97.805038) (width 0.2) (layer "F.Cu") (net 5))
 (segment (start 123.32 97.805038) (end 123.32 97.830343) (width 0.2) (layer "F.Cu") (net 5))
 (segment (start 119.38 95.540343) (end 119.45 95.610343) (width 0.2) (layer "F.Cu") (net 5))
 (segment (start 119.38 91.722843) (end 119.38 95.540343) (width 0.2) (layer "F.Cu") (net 5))
 (segment (start 120.50104 96.410343) (end 117.005686 96.410343) (width 0.2) (layer "F.Cu") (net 3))
 (segment (start 121.32 97.830343) (end 121.32 97.229303) (width 0.2) (layer "F.Cu") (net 3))
 (segment (start 121.32 97.229303) (end 120.50104 96.410343) (width 0.2) (layer "F.Cu") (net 3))
 (segment (start 117.005686 96.410343) (end 116.84 96.244657) (width 0.2) (layer "F.Cu") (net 3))
 (segment (start 116.84 96.244657) (end 116.84 94.262843) (width 0.2) (layer "F.Cu") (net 3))
 (segment (start 116.84 94.262843) (end 114.3 91.722843) (width 0.2) (layer "F.Cu") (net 3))
 (segment (start 132.49896 77.720343) (end 133.1 77.720343) (width 0.2) (layer "F.Cu") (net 7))
 (segment (start 125.5425 84.676803) (end 132.49896 77.720343) (width 0.2) (layer "F.Cu") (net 7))
 (segment (start 125.5425 90.640343) (end 125.5425 84.676803) (width 0.2) (layer "F.Cu") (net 7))
 (segment (start 124.46 91.722843) (end 125.5425 90.640343) (width 0.2) (layer "F.Cu") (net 7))
 (segment (start 119.3 96.810343) (end 116.84 96.810343) (width 0.2) (layer "F.Cu") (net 2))
 (segment (start 114.035 93.997843) (end 111.76 91.722843) (width 0.2) (layer "F.Cu") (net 2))
 (segment (start 116.84 96.810343) (end 116.605686 96.576028) (width 0.2) (layer "F.Cu") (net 2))
 (segment (start 120.32 97.830343) (end 119.3 96.810343) (width 0.2) (layer "F.Cu") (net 2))
 (segment (start 116.605686 96.576028) (end 116.44 96.410343) (width 0.2) (layer "F.Cu") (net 2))
 (segment (start 116.009314 93.997843) (end 114.035 93.997843) (width 0.2) (layer "F.Cu") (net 2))
 (segment (start 116.44 94.428529) (end 116.009314 93.997843) (width 0.2) (layer "F.Cu") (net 2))
 (segment (start 116.44 96.410343) (end 116.44 94.428529) (width 0.2) (layer "F.Cu") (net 2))
 (segment (start 127.41792 82.235697) (end 132.933274 76.720343) (width 0.2) (layer "F.Cu") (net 8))
 (segment (start 132.933274 76.720343) (end 133.1 76.720343) (width 0.2) (layer "F.Cu") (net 8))
 (segment (start 125.094314 82.235697) (end 127.41792 82.235697) (width 0.2) (layer "F.Cu") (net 8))
 (segment (start 124.46 75.697843) (end 124.46 81.601383) (width 0.2) (layer "F.Cu") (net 8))
 (segment (start 124.46 81.601383) (end 125.094314 82.235697) (width 0.2) (layer "F.Cu") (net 8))
 (segment (start 109.22 94.270343) (end 105.41 90.460343) (width 0.2) (layer "F.Cu") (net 18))
 (segment (start 113.76 97.229303) (end 110.80104 94.270343) (width 0.2) (layer "F.Cu") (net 18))
 (segment (start 118.145001 67.925344) (end 117.264999 67.925344) (width 0.2) (layer "F.Cu") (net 18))
 (segment (start 112.56 70.940343) (end 116.896726 70.940343) (width 0.2) (layer "F.Cu") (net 18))
 (segment (start 118.57 69.267069) (end 118.57 68.350343) (width 0.2) (layer "F.Cu") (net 18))
 (segment (start 117.264999 67.925344) (end 116.84 68.350343) (width 0.2) (layer "F.Cu") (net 18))
 (segment (start 110.80104 94.270343) (end 109.22 94.270343) (width 0.2) (layer "F.Cu") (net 18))
 (segment (start 110.49 68.870343) (end 112.56 70.940343) (width 0.2) (layer "F.Cu") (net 18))
 (segment (start 105.41 68.870343) (end 110.49 68.870343) (width 0.2) (layer "F.Cu") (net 18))
 (segment (start 105.41 90.460343) (end 105.41 68.870343) (width 0.2) (layer "F.Cu") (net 18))
 (segment (start 118.57 68.350343) (end 118.145001 67.925344) (width 0.2) (layer "F.Cu") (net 18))
 (segment (start 113.76 97.830343) (end 113.76 97.229303) (width 0.2) (layer "F.Cu") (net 18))
 (segment (start 116.896726 70.940343) (end 118.57 69.267069) (width 0.2) (layer "F.Cu") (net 18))
 (segment (start 133.1 85.320343) (end 133.1 82.880343) (width 0.2) (layer "B.Cu") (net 18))
 (segment (start 133.1 82.880343) (end 118.57 68.350343) (width 0.2) (layer "B.Cu") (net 18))
 (segment (start 118.57 68.350343) (end 116.84 68.350343) (width 0.2) (layer "B.Cu") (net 18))
 (segment (start 105.01 91.330343) (end 105.01 68.704658) (width 0.2) (layer "F.Cu") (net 17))
 (segment (start 108.4775 94.797843) (end 105.01 91.330343) (width 0.2) (layer "F.Cu") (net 17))
 (segment (start 111.36 68.470343) (end 113.43 70.540343) (width 0.2) (layer "F.Cu") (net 17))
 (segment (start 115.84 70.270343) (end 115.57 70.540343) (width 0.2) (layer "F.Cu") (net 17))
 (segment (start 112.76 97.830343) (end 112.76 97.229303) (width 0.2) (layer "F.Cu") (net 17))
 (segment (start 105.01 68.704658) (end 105.244315 68.470343) (width 0.2) (layer "F.Cu") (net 17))
 (segment (start 105.244315 68.470343) (end 111.36 68.470343) (width 0.2) (layer "F.Cu") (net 17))
 (segment (start 112.504645 97.229303) (end 110.073185 94.797843) (width 0.2) (layer "F.Cu") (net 17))
 (segment (start 112.76 97.229303) (end 112.504645 97.229303) (width 0.2) (layer "F.Cu") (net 17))
 (segment (start 115.84 68.350343) (end 115.84 70.270343) (width 0.2) (layer "F.Cu") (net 17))
 (segment (start 113.43 70.540343) (end 115.57 70.540343) (width 0.2) (layer "F.Cu") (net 17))
 (segment (start 110.073185 94.797843) (end 108.4775 94.797843) (width 0.2) (layer "F.Cu") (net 17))
 (segment (start 133.1 86.320343) (end 133.02 86.320343) (width 0.2) (layer "B.Cu") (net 17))
 (segment (start 133.02 86.320343) (end 115.84 69.140343) (width 0.2) (layer "B.Cu") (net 17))
 (segment (start 115.84 69.140343) (end 115.84 68.350343) (width 0.2) (layer "B.Cu") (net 17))
 (via (at 109.22 90.460343) (size 0.6) (drill 0.3) (layers "F.Cu" "B.Cu") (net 1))
 (segment (start 115.57 72.680343) (end 113.84 70.950343) (width 0.2) (layer "B.Cu") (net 1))
 (segment (start 113.84 70.950343) (end 113.84 68.350343) (width 0.2) (layer "B.Cu") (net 1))
 (segment (start 115.57 72.680343) (end 115.57 84.110343) (width 0.2) (layer "B.Cu") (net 1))
 (segment (start 115.57 84.110343) (end 109.22 90.460343) (width 0.2) (layer "B.Cu") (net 1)))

